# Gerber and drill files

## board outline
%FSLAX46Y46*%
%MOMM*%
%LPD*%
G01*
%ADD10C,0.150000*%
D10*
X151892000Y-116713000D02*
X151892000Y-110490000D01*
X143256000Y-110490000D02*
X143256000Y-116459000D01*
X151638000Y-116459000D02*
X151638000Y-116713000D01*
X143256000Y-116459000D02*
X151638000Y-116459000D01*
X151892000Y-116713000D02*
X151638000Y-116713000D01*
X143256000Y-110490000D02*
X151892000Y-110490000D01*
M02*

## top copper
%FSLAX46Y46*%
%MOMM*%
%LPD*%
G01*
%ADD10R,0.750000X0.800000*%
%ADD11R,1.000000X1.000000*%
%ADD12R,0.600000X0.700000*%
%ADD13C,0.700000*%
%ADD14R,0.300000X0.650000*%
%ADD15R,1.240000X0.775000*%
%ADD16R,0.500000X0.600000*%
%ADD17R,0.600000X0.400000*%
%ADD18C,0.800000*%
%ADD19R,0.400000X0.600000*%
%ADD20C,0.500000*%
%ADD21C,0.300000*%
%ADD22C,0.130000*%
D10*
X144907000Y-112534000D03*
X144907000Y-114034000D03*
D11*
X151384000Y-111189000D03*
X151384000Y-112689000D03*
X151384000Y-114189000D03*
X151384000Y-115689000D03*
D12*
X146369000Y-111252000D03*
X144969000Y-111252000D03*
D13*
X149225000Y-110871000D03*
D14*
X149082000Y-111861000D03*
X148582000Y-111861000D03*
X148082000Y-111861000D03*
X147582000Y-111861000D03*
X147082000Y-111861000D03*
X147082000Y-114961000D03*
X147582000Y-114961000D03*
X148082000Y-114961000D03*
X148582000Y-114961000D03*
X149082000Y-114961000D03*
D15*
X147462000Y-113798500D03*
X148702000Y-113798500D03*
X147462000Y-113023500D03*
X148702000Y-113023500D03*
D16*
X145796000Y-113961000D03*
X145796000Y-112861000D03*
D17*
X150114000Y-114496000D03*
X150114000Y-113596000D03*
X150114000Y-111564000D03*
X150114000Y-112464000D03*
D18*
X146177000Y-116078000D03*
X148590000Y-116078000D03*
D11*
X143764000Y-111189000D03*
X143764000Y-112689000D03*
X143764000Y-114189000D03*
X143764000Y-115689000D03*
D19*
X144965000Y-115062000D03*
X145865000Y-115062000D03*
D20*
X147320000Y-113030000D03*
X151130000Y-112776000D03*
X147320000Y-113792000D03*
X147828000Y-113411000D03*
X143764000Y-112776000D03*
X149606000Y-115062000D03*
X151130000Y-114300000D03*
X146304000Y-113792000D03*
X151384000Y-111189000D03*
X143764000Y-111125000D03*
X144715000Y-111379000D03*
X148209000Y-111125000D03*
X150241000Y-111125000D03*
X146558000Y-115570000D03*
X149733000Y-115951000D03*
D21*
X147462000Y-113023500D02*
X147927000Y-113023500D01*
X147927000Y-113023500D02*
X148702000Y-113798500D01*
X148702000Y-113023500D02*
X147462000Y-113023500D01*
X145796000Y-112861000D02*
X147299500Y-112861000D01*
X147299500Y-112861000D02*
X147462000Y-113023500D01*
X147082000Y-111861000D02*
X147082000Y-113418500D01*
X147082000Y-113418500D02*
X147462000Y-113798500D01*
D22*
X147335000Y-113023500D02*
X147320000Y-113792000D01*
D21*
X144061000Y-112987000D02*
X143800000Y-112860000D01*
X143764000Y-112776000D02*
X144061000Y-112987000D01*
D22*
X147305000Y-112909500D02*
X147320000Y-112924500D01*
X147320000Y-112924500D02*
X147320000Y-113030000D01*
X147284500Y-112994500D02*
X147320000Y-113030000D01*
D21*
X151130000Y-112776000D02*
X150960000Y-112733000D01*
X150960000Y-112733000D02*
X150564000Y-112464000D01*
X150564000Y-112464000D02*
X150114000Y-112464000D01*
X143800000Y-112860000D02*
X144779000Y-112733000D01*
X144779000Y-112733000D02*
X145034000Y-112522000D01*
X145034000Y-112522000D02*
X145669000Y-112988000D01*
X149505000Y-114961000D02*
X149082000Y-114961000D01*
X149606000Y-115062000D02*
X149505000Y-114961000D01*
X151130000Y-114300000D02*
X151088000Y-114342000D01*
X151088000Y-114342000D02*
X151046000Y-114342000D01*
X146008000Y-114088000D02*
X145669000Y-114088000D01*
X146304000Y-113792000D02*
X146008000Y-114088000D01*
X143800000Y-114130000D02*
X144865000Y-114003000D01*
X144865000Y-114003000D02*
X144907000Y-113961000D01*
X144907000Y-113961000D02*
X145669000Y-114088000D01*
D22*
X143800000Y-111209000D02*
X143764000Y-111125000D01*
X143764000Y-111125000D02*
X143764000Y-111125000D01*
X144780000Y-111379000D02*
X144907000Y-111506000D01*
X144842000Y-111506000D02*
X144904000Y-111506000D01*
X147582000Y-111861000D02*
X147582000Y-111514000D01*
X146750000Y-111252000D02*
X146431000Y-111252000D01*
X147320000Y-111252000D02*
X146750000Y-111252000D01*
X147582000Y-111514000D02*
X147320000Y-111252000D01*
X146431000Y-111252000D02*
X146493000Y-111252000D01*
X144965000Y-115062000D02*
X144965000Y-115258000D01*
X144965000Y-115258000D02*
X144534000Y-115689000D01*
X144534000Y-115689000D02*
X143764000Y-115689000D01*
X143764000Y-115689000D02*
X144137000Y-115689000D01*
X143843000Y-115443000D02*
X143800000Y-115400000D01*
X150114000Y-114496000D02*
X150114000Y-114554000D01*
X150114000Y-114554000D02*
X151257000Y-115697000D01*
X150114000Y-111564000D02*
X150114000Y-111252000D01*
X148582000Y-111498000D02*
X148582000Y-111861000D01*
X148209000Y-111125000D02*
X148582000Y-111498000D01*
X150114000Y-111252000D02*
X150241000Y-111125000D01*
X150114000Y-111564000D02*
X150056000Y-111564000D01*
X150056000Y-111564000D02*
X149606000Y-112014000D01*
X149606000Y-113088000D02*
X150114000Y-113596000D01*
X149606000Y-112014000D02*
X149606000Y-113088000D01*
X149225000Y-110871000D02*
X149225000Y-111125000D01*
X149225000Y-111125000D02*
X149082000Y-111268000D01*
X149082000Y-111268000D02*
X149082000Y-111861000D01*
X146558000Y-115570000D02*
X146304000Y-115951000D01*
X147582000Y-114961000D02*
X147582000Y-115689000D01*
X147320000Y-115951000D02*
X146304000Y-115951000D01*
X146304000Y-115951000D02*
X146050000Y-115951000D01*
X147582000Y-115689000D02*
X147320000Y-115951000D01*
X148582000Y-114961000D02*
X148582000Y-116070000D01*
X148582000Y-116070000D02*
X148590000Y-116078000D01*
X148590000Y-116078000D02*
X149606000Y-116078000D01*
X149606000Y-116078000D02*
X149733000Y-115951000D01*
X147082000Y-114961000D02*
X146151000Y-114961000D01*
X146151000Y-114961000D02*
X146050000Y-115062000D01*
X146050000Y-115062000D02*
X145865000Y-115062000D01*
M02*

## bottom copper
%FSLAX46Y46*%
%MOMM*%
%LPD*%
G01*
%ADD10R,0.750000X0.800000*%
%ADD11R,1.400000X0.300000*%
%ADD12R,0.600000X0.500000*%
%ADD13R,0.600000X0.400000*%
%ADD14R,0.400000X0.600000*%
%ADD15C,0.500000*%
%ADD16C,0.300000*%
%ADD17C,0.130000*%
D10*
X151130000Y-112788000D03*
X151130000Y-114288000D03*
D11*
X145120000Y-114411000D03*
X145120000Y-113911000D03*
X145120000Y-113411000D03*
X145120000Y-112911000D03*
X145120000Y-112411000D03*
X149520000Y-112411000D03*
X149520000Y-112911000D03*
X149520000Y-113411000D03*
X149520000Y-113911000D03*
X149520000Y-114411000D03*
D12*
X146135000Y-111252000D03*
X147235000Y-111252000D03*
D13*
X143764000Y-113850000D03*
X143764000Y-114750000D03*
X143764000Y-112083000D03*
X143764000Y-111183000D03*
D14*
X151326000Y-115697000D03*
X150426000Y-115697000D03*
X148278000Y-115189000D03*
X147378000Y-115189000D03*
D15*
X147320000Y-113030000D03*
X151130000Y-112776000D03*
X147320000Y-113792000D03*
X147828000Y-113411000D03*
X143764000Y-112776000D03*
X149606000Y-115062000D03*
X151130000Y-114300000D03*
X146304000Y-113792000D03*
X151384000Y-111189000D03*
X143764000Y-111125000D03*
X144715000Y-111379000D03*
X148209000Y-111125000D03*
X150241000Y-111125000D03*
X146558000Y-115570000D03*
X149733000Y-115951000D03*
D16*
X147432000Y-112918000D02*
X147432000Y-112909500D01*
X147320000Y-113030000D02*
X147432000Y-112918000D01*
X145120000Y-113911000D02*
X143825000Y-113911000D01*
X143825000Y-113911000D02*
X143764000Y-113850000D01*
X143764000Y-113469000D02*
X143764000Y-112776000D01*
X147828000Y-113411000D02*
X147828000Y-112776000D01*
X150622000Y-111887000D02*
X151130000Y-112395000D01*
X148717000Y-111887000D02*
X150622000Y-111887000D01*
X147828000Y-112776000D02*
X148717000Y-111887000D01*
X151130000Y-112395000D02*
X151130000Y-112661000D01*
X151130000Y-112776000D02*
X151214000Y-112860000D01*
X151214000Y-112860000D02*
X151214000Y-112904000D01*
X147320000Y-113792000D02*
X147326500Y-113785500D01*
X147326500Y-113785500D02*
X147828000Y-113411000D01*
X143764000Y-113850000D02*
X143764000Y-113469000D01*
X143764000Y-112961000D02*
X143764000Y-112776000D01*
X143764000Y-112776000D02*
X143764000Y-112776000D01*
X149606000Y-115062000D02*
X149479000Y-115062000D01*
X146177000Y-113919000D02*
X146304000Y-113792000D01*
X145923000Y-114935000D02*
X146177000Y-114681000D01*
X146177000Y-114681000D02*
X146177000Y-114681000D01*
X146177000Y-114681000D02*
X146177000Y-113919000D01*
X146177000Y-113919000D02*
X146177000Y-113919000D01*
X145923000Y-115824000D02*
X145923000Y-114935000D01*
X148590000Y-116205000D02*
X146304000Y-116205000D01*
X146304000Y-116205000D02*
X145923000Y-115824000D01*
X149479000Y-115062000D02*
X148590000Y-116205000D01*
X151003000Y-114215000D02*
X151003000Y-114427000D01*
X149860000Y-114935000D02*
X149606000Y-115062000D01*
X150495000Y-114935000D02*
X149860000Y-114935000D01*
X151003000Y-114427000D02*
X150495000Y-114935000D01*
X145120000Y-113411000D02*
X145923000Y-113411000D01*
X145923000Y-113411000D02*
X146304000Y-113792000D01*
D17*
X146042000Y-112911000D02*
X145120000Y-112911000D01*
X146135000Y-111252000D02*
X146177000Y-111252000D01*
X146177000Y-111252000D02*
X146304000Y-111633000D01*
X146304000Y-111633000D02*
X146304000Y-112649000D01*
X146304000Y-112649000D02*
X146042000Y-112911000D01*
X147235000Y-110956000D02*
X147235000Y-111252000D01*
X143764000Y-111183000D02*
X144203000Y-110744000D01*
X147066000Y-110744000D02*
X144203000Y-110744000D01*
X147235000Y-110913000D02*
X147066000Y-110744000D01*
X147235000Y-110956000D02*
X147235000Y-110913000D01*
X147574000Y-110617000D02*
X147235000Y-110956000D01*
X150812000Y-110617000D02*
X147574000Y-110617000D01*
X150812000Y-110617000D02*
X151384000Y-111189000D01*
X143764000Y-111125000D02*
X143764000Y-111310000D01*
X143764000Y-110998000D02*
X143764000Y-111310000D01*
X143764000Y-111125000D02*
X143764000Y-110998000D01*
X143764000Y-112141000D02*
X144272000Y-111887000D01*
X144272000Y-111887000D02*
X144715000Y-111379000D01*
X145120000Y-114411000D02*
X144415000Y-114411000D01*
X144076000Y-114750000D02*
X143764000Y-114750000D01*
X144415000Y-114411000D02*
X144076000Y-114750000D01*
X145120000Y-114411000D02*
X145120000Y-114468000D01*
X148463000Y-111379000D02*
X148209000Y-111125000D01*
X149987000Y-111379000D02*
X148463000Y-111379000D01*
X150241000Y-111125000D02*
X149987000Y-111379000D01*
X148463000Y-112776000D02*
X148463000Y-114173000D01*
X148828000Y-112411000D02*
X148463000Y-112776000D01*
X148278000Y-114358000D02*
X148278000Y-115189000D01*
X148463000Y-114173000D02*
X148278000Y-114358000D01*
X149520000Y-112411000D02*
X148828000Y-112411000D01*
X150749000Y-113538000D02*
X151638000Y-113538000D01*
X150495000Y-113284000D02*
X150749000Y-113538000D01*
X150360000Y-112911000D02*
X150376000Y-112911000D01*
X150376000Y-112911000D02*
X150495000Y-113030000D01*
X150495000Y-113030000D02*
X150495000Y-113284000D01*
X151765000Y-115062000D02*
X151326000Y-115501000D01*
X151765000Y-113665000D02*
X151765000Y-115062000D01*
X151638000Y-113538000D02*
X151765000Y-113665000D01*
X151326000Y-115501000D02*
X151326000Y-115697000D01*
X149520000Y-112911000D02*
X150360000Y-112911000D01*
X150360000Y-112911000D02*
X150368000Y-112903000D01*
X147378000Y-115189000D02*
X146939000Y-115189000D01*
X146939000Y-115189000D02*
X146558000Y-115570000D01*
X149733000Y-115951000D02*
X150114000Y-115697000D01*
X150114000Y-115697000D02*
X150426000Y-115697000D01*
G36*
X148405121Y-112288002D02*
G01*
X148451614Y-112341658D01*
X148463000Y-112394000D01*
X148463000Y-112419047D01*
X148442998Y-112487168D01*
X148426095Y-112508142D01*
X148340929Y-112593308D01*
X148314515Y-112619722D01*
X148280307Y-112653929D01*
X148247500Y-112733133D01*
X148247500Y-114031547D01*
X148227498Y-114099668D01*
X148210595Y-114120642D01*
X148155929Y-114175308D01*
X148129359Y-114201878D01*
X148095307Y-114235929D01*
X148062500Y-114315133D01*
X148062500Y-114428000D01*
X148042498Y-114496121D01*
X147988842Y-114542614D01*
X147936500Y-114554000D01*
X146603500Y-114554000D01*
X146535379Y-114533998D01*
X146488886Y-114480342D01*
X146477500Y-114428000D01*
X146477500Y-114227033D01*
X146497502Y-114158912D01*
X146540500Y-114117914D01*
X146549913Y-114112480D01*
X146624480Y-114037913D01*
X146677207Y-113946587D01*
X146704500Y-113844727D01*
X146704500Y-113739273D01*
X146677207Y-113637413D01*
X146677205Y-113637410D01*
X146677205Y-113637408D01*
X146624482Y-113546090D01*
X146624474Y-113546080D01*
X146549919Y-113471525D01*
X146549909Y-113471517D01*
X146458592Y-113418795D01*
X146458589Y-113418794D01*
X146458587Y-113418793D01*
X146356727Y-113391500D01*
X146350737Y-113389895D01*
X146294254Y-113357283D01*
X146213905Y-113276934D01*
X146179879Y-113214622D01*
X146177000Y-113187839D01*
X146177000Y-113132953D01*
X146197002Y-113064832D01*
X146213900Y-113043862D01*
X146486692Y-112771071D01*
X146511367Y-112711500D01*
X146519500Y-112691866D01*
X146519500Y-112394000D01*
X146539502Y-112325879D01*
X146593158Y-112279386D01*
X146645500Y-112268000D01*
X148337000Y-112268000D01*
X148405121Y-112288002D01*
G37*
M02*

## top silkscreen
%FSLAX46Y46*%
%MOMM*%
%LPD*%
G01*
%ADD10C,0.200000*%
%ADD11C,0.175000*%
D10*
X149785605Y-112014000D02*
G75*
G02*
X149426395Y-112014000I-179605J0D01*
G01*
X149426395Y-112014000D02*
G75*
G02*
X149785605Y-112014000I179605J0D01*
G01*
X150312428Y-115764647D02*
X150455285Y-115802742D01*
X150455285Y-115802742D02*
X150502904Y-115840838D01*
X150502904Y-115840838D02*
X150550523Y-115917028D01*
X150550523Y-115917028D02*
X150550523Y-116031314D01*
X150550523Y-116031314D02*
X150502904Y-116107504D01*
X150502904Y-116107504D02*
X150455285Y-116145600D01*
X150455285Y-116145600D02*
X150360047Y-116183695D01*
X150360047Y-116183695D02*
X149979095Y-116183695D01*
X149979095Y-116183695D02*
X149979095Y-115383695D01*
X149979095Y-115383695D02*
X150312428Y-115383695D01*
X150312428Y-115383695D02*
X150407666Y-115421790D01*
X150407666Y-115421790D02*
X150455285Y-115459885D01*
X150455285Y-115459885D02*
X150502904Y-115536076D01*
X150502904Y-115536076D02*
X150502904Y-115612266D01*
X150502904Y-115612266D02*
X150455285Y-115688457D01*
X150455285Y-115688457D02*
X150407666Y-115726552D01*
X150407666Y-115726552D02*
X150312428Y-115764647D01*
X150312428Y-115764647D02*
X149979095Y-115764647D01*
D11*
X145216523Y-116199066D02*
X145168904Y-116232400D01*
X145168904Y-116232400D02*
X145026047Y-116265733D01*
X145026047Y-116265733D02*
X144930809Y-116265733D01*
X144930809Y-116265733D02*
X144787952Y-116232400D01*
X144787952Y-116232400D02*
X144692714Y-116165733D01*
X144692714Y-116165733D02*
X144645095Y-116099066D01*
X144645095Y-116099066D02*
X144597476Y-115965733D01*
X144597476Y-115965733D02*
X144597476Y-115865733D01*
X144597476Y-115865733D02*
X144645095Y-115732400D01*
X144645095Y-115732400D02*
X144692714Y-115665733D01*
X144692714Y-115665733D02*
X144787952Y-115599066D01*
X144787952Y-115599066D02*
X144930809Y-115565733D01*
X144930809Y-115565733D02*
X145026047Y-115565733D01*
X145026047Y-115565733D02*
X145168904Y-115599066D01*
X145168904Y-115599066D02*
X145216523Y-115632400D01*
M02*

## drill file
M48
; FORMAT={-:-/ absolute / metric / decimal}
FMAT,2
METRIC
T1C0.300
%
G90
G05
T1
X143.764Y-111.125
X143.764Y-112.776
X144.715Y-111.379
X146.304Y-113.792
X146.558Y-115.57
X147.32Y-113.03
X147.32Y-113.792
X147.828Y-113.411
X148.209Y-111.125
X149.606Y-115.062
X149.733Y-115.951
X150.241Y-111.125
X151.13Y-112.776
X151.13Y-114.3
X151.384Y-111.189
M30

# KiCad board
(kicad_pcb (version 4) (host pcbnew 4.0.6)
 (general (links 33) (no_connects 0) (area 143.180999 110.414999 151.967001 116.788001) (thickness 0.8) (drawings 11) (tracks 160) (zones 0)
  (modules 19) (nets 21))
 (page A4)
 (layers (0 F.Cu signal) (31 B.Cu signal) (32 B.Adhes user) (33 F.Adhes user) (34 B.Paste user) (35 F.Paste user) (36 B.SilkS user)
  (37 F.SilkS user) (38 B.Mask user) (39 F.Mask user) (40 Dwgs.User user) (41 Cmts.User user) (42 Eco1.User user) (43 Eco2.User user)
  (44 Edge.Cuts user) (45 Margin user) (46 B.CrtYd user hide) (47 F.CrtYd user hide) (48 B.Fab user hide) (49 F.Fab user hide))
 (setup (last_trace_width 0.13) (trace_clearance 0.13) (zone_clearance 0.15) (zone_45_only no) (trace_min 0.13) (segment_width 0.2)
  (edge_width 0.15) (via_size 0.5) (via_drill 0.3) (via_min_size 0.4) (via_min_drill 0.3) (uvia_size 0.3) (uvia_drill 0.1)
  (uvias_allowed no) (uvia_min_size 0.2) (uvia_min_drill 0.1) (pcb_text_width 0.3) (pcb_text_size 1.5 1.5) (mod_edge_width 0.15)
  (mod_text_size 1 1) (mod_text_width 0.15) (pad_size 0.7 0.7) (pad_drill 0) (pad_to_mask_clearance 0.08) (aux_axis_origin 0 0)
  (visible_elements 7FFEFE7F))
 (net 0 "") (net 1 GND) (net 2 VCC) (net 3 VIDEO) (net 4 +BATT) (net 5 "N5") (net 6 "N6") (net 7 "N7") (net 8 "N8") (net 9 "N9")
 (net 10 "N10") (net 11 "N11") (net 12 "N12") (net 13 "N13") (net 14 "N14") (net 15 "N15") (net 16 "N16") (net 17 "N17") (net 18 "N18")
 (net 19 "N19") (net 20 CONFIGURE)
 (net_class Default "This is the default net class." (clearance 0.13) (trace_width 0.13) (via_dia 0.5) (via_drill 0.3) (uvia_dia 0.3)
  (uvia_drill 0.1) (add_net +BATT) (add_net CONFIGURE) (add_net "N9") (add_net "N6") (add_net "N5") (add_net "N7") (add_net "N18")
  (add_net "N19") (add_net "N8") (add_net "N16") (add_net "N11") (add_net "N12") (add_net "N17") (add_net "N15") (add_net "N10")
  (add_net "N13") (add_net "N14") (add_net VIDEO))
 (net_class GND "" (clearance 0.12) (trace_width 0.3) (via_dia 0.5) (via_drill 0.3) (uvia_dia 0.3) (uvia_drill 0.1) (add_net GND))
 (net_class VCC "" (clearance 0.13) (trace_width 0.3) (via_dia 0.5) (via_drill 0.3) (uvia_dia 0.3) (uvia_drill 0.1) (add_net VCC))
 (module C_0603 (layer B.Cu) (at 151.13 113.538 270)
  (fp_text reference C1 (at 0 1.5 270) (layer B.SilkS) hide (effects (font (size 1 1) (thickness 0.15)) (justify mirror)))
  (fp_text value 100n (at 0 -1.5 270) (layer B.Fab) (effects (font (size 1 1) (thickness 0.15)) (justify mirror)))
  (pad 1 smd rect (at -0.75 0 270) (size 0.8 0.75) (layers B.Cu B.Paste B.Mask) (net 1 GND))
  (pad 2 smd rect (at 0.75 0 270) (size 0.8 0.75) (layers B.Cu B.Paste B.Mask) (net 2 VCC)))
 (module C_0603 (layer F.Cu) (at 144.907 113.284 270)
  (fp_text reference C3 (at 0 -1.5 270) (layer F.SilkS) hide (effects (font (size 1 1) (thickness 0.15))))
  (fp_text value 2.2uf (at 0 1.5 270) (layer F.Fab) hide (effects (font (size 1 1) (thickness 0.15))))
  (pad 1 smd rect (at -0.75 0 270) (size 0.8 0.75) (layers F.Cu F.Paste F.Mask) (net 1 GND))
  (pad 2 smd rect (at 0.75 0 270) (size 0.8 0.75) (layers F.Cu F.Paste F.Mask) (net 2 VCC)))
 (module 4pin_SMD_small (layer F.Cu) (at 151.384 115.189 90)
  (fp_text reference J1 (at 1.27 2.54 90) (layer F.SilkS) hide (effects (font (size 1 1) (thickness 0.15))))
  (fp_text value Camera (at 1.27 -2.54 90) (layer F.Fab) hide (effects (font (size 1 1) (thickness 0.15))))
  (pad 4 smd rect (at 4 0 90) (size 1 1) (layers F.Cu F.Paste F.Mask) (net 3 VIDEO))
  (pad 3 smd rect (at 2.5 0 90) (size 1 1) (layers F.Cu F.Paste F.Mask) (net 1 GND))
  (pad 2 smd rect (at 1 0 90) (size 1 1) (layers F.Cu F.Paste F.Mask) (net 2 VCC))
  (pad 1 smd rect (at -0.5 0 90) (size 1 1) (layers F.Cu F.Paste F.Mask) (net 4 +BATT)))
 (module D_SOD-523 (layer F.Cu) (at 145.669 111.252)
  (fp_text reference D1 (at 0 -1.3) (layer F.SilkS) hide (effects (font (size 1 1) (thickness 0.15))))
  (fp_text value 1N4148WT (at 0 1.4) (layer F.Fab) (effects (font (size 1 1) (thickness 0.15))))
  (pad 2 smd rect (at 0.7 0 180) (size 0.6 0.7) (layers F.Cu F.Paste F.Mask) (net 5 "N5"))
  (pad 1 smd rect (at -0.7 0 180) (size 0.6 0.7) (layers F.Cu F.Paste F.Mask) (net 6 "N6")))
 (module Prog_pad (layer F.Cu) (at 149.225 110.871)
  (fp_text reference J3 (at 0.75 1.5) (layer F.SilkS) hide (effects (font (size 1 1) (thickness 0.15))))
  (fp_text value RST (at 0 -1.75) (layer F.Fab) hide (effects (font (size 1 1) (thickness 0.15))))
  (pad 1 smd circle (at 0 0) (size 0.7 0.7) (layers F.Cu F.Paste F.Mask) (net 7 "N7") (solder_mask_margin 0.02)))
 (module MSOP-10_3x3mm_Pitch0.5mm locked (layer B.Cu) (at 147.32 113.411)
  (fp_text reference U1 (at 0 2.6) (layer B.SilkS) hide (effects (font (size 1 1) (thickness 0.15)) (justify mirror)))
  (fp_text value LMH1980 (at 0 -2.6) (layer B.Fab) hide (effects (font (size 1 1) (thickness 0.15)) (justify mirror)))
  (pad 1 smd rect (at -2.2 1) (size 1.4 0.3) (layers B.Cu B.Paste B.Mask) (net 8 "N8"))
  (pad 2 smd rect (at -2.2 0.5) (size 1.4 0.3) (layers B.Cu B.Paste B.Mask) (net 1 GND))
  (pad 3 smd rect (at -2.2 0) (size 1.4 0.3) (layers B.Cu B.Paste B.Mask) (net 2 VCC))
  (pad 4 smd rect (at -2.2 -0.5) (size 1.4 0.3) (layers B.Cu B.Paste B.Mask) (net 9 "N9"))
  (pad 5 smd rect (at -2.2 -1) (size 1.4 0.3) (layers B.Cu B.Paste B.Mask) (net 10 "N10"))
  (pad 6 smd rect (at 2.2 -1) (size 1.4 0.3) (layers B.Cu B.Paste B.Mask) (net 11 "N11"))
  (pad 7 smd rect (at 2.2 -0.5) (size 1.4 0.3) (layers B.Cu B.Paste B.Mask) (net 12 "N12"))
  (pad 8 smd rect (at 2.2 0) (size 1.4 0.3) (layers B.Cu B.Paste B.Mask) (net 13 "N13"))
  (pad 9 smd rect (at 2.2 0.5) (size 1.4 0.3) (layers B.Cu B.Paste B.Mask) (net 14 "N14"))
  (pad 10 smd rect (at 2.2 1) (size 1.4 0.3) (layers B.Cu B.Paste B.Mask) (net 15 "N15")))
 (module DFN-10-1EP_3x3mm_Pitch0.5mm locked (layer F.Cu) (at 148.082 113.411 270)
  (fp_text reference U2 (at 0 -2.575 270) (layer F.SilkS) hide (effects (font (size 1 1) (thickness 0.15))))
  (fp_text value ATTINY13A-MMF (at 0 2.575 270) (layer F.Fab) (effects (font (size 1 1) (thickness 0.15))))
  (pad 1 smd rect (at -1.55 -1 270) (size 0.65 0.3) (layers F.Cu F.Paste F.Mask) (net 7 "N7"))
  (pad 2 smd rect (at -1.55 -0.5 270) (size 0.65 0.3) (layers F.Cu F.Paste F.Mask) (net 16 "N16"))
  (pad 3 smd rect (at -1.55 0 270) (size 0.65 0.3) (layers F.Cu F.Paste F.Mask))
  (pad 4 smd rect (at -1.55 0.5 270) (size 0.65 0.3) (layers F.Cu F.Paste F.Mask) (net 5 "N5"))
  (pad 5 smd rect (at -1.55 1 270) (size 0.65 0.3) (layers F.Cu F.Paste F.Mask) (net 1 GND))
  (pad 6 smd rect (at 1.55 1 270) (size 0.65 0.3) (layers F.Cu F.Paste F.Mask) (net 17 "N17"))
  (pad 7 smd rect (at 1.55 0.5 270) (size 0.65 0.3) (layers F.Cu F.Paste F.Mask) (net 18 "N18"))
  (pad 8 smd rect (at 1.55 0 270) (size 0.65 0.3) (layers F.Cu F.Paste F.Mask))
  (pad 9 smd rect (at 1.55 -0.5 270) (size 0.65 0.3) (layers F.Cu F.Paste F.Mask) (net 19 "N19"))
  (pad 10 smd rect (at 1.55 -1 270) (size 0.65 0.3) (layers F.Cu F.Paste F.Mask) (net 2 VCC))
  (pad 11 smd rect (at 0.3875 0.62 270) (size 0.775 1.24) (layers F.Cu F.Paste F.Mask) (solder_paste_margin_ratio -0.2))
  (pad 11 smd rect (at 0.3875 -0.62 270) (size 0.775 1.24) (layers F.Cu F.Paste F.Mask) (solder_paste_margin_ratio -0.2))
  (pad 11 smd rect (at -0.3875 0.62 270) (size 0.775 1.24) (layers F.Cu F.Paste F.Mask) (solder_paste_margin_ratio -0.2))
  (pad 11 smd rect (at -0.3875 -0.62 270) (size 0.775 1.24) (layers F.Cu F.Paste F.Mask) (solder_paste_margin_ratio -0.2)))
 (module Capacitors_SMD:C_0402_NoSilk (layer B.Cu) (at 146.685 111.252)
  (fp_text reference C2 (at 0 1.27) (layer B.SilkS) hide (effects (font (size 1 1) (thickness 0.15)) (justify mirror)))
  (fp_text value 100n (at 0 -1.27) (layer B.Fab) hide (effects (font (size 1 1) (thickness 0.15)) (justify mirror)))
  (pad 1 smd rect (at -0.55 0) (size 0.6 0.5) (layers B.Cu B.Paste B.Mask) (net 9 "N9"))
  (pad 2 smd rect (at 0.55 0) (size 0.6 0.5) (layers B.Cu B.Paste B.Mask) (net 3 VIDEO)))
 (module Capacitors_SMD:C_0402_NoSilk (layer F.Cu) (at 145.796 113.411 90)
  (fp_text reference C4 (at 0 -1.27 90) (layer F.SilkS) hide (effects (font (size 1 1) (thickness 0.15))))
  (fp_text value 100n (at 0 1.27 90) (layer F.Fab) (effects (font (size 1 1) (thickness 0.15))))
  (pad 1 smd rect (at -0.55 0 90) (size 0.6 0.5) (layers F.Cu F.Paste F.Mask) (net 2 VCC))
  (pad 2 smd rect (at 0.55 0 90) (size 0.6 0.5) (layers F.Cu F.Paste F.Mask) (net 1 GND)))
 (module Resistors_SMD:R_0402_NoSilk (layer B.Cu) (at 143.764 114.3 270)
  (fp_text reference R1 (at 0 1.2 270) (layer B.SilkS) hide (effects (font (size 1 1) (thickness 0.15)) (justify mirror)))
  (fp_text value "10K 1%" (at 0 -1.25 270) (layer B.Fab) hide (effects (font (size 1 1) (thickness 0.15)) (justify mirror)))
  (pad 1 smd rect (at -0.45 0 270) (size 0.4 0.6) (layers B.Cu B.Paste B.Mask) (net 1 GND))
  (pad 2 smd rect (at 0.45 0 270) (size 0.4 0.6) (layers B.Cu B.Paste B.Mask) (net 8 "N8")))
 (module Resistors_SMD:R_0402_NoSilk (layer B.Cu) (at 143.764 111.633 90)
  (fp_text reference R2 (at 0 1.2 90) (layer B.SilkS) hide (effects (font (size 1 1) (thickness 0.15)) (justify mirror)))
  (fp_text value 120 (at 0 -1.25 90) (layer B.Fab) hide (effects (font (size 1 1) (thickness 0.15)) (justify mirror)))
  (pad 1 smd rect (at -0.45 0 90) (size 0.4 0.6) (layers B.Cu B.Paste B.Mask) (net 6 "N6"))
  (pad 2 smd rect (at 0.45 0 90) (size 0.4 0.6) (layers B.Cu B.Paste B.Mask) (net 3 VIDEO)))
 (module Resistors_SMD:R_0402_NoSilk (layer F.Cu) (at 150.114 114.046 90)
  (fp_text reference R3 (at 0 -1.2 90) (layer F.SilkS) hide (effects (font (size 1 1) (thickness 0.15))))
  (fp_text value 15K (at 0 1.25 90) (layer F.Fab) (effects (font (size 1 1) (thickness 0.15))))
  (pad 1 smd rect (at -0.45 0 90) (size 0.4 0.6) (layers F.Cu F.Paste F.Mask) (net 4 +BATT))
  (pad 2 smd rect (at 0.45 0 90) (size 0.4 0.6) (layers F.Cu F.Paste F.Mask) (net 16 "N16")))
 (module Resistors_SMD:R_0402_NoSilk (layer F.Cu) (at 150.114 112.014 270)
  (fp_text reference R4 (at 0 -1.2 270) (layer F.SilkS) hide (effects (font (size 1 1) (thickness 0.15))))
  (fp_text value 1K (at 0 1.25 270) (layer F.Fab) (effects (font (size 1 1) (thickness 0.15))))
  (pad 1 smd rect (at -0.45 0 270) (size 0.4 0.6) (layers F.Cu F.Paste F.Mask) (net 16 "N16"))
  (pad 2 smd rect (at 0.45 0 270) (size 0.4 0.6) (layers F.Cu F.Paste F.Mask) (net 1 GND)))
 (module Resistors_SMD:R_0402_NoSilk (layer B.Cu) (at 150.876 115.697 180)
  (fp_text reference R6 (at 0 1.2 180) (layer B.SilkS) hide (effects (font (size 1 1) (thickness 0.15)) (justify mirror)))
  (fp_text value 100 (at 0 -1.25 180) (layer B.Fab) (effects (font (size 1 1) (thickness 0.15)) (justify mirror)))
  (pad 1 smd rect (at -0.45 0 180) (size 0.4 0.6) (layers B.Cu B.Paste B.Mask) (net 12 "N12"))
  (pad 2 smd rect (at 0.45 0 180) (size 0.4 0.6) (layers B.Cu B.Paste B.Mask) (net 19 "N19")))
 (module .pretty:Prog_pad (layer F.Cu) (at 146.177 116.078)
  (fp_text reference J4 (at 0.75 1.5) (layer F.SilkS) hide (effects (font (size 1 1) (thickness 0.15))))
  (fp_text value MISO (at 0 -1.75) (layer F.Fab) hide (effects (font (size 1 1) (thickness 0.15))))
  (pad 1 smd circle (at 0 0) (size 0.8 0.8) (layers F.Cu F.Paste F.Mask) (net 18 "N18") (solder_mask_margin 0.02)))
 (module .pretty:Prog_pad (layer F.Cu) (at 148.59 116.078)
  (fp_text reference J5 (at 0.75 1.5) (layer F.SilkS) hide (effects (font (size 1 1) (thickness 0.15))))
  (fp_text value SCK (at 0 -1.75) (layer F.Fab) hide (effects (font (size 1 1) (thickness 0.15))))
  (pad 1 smd circle (at 0 0) (size 0.8 0.8) (layers F.Cu F.Paste F.Mask) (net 19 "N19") (solder_mask_margin 0.02)))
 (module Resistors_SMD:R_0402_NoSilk (layer B.Cu) (at 147.828 115.189 180)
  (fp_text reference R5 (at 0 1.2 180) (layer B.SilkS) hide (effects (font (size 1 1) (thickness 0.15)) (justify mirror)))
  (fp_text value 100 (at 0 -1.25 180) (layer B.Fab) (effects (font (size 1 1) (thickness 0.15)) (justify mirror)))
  (pad 1 smd rect (at -0.45 0 180) (size 0.4 0.6) (layers B.Cu B.Paste B.Mask) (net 11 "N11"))
  (pad 2 smd rect (at 0.45 0 180) (size 0.4 0.6) (layers B.Cu B.Paste B.Mask) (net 18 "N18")))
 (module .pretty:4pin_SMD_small (layer F.Cu) (at 143.764 115.189 90)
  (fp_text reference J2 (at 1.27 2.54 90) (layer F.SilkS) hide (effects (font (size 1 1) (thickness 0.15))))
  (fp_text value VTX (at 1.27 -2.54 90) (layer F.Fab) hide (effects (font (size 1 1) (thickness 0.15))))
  (pad 4 smd rect (at 4 0 90) (size 1 1) (layers F.Cu F.Paste F.Mask) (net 3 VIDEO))
  (pad 3 smd rect (at 2.5 0 90) (size 1 1) (layers F.Cu F.Paste F.Mask) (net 1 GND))
  (pad 2 smd rect (at 1 0 90) (size 1 1) (layers F.Cu F.Paste F.Mask) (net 2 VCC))
  (pad 1 smd rect (at -0.5 0 90) (size 1 1) (layers F.Cu F.Paste F.Mask) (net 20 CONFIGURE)))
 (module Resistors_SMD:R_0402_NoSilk (layer F.Cu) (at 145.415 115.062)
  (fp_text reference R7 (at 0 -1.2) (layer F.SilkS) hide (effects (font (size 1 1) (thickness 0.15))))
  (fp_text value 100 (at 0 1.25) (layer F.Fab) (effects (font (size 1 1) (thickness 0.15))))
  (pad 1 smd rect (at -0.45 0) (size 0.4 0.6) (layers F.Cu F.Paste F.Mask) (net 20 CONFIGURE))
  (pad 2 smd rect (at 0.45 0) (size 0.4 0.6) (layers F.Cu F.Paste F.Mask) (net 17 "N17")))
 (gr_line (start 151.892 116.713) (end 151.892 110.49) (angle 90) (layer Edge.Cuts) (width 0.15))
 (gr_line (start 143.256 110.49) (end 143.256 116.459) (angle 90) (layer Edge.Cuts) (width 0.15))
 (gr_line (start 151.638 116.459) (end 151.638 116.713) (angle 90) (layer Edge.Cuts) (width 0.15))
 (gr_line (start 143.256 116.459) (end 151.638 116.459) (angle 90) (layer Edge.Cuts) (width 0.15))
 (gr_line (start 151.892 116.713) (end 151.638 116.713) (angle 90) (layer Edge.Cuts) (width 0.15))
 (gr_circle (center 149.606 112.014) (end 149.479 111.887) (layer F.SilkS) (width 0.2))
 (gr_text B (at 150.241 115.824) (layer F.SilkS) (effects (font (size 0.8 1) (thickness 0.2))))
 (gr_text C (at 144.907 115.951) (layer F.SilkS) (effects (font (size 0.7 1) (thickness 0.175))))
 (gr_line (start 143.256 110.49) (end 151.892 110.49) (angle 90) (layer Edge.Cuts) (width 0.15))
 (segment (start 147.462 113.0235) (end 147.927 113.0235) (width 0.3) (layer F.Cu) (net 1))
 (segment (start 147.927 113.0235) (end 148.702 113.7985) (width 0.3) (layer F.Cu) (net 1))
 (segment (start 148.702 113.0235) (end 147.462 113.0235) (width 0.3) (layer F.Cu) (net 1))
 (segment (start 145.796 112.861) (end 147.2995 112.861) (width 0.3) (layer F.Cu) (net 1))
 (segment (start 147.2995 112.861) (end 147.462 113.0235) (width 0.3) (layer F.Cu) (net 1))
 (segment (start 147.082 111.861) (end 147.082 113.4185) (width 0.3) (layer F.Cu) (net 1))
 (segment (start 147.082 113.4185) (end 147.462 113.7985) (width 0.3) (layer F.Cu) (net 1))
 (via (at 147.32 113.03) (size 0.5) (drill 0.3) (layers F.Cu B.Cu) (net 1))
 (segment (start 147.432 112.918) (end 147.432 112.9095) (width 0.3) (layer B.Cu) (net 1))
 (segment (start 147.32 113.03) (end 147.432 112.918) (width 0.3) (layer B.Cu) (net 1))
 (segment (start 145.12 113.911) (end 143.825 113.911) (width 0.3) (layer B.Cu) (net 1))
 (segment (start 143.825 113.911) (end 143.764 113.85) (width 0.3) (layer B.Cu) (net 1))
 (segment (start 143.764 113.469) (end 143.764 112.776) (width 0.3) (layer B.Cu) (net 1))
 (segment (start 147.828 113.411) (end 147.828 112.776) (width 0.3) (layer B.Cu) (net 1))
 (segment (start 150.622 111.887) (end 151.13 112.395) (width 0.3) (layer B.Cu) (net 1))
 (segment (start 148.717 111.887) (end 150.622 111.887) (width 0.3) (layer B.Cu) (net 1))
 (segment (start 147.828 112.776) (end 148.717 111.887) (width 0.3) (layer B.Cu) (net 1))
 (segment (start 151.13 112.395) (end 151.13 112.661) (width 0.3) (layer B.Cu) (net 1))
 (via (at 151.13 112.776) (size 0.5) (drill 0.3) (layers F.Cu B.Cu) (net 1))
 (segment (start 151.13 112.776) (end 151.214 112.86) (width 0.3) (layer B.Cu) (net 1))
 (segment (start 151.214 112.86) (end 151.214 112.904) (width 0.3) (layer B.Cu) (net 1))
 (segment (start 147.335 113.0235) (end 147.32 113.792) (width 0.13) (layer F.Cu) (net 1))
 (via (at 147.32 113.792) (size 0.5) (drill 0.3) (layers F.Cu B.Cu) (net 1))
 (segment (start 147.32 113.792) (end 147.3265 113.7855) (width 0.3) (layer B.Cu) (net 1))
 (segment (start 147.3265 113.7855) (end 147.828 113.411) (width 0.3) (layer B.Cu) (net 1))
 (via (at 147.828 113.411) (size 0.5) (drill 0.3) (layers F.Cu B.Cu) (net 1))
 (segment (start 143.764 113.85) (end 143.764 113.469) (width 0.3) (layer B.Cu) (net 1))
 (segment (start 143.764 112.961) (end 143.764 112.776) (width 0.3) (layer B.Cu) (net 1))
 (segment (start 144.061 112.987) (end 143.8 112.86) (width 0.3) (layer F.Cu) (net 1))
 (segment (start 143.764 112.776) (end 144.061 112.987) (width 0.3) (layer F.Cu) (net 1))
 (via (at 143.764 112.776) (size 0.5) (drill 0.3) (layers F.Cu B.Cu) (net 1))
 (segment (start 143.764 112.776) (end 143.764 112.776) (width 0.3) (layer B.Cu) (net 1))
 (segment (start 147.305 112.9095) (end 147.32 112.9245) (width 0.13) (layer F.Cu) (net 1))
 (segment (start 147.32 112.9245) (end 147.32 113.03) (width 0.13) (layer F.Cu) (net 1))
 (segment (start 147.2845 112.9945) (end 147.32 113.03) (width 0.13) (layer F.Cu) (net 1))
 (segment (start 151.13 112.776) (end 150.96 112.733) (width 0.3) (layer F.Cu) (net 1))
 (segment (start 150.96 112.733) (end 150.564 112.464) (width 0.3) (layer F.Cu) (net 1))
 (segment (start 150.564 112.464) (end 150.114 112.464) (width 0.3) (layer F.Cu) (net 1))
 (segment (start 143.8 112.86) (end 144.779 112.733) (width 0.3) (layer F.Cu) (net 1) (status 20))
 (segment (start 144.779 112.733) (end 145.034 112.522) (width 0.3) (layer F.Cu) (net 1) (status 30))
 (segment (start 145.034 112.522) (end 145.669 112.988) (width 0.3) (layer F.Cu) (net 1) (status 10))
 (segment (start 149.606 115.062) (end 149.479 115.062) (width 0.3) (layer B.Cu) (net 2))
 (segment (start 146.177 113.919) (end 146.304 113.792) (width 0.3) (layer B.Cu) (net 2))
 (segment (start 145.923 114.935) (end 146.177 114.681) (width 0.3) (layer B.Cu) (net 2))
 (segment (start 146.177 114.681) (end 146.177 114.681) (width 0.3) (layer B.Cu) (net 2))
 (segment (start 146.177 114.681) (end 146.177 113.919) (width 0.3) (layer B.Cu) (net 2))
 (segment (start 146.177 113.919) (end 146.177 113.919) (width 0.3) (layer B.Cu) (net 2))
 (segment (start 145.923 115.824) (end 145.923 114.935) (width 0.3) (layer B.Cu) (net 2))
 (segment (start 148.59 116.205) (end 146.304 116.205) (width 0.3) (layer B.Cu) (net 2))
 (segment (start 146.304 116.205) (end 145.923 115.824) (width 0.3) (layer B.Cu) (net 2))
 (segment (start 149.479 115.062) (end 148.59 116.205) (width 0.3) (layer B.Cu) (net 2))
 (segment (start 151.003 114.215) (end 151.003 114.427) (width 0.3) (layer B.Cu) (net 2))
 (segment (start 149.505 114.961) (end 149.082 114.961) (width 0.3) (layer F.Cu) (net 2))
 (segment (start 149.606 115.062) (end 149.505 114.961) (width 0.3) (layer F.Cu) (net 2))
 (via (at 149.606 115.062) (size 0.5) (drill 0.3) (layers F.Cu B.Cu) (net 2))
 (segment (start 149.86 114.935) (end 149.606 115.062) (width 0.3) (layer B.Cu) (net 2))
 (segment (start 150.495 114.935) (end 149.86 114.935) (width 0.3) (layer B.Cu) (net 2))
 (segment (start 151.003 114.427) (end 150.495 114.935) (width 0.3) (layer B.Cu) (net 2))
 (via (at 151.13 114.3) (size 0.5) (drill 0.3) (layers F.Cu B.Cu) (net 2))
 (segment (start 151.13 114.3) (end 151.088 114.342) (width 0.3) (layer F.Cu) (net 2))
 (segment (start 151.088 114.342) (end 151.046 114.342) (width 0.3) (layer F.Cu) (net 2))
 (segment (start 145.12 113.411) (end 145.923 113.411) (width 0.3) (layer B.Cu) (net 2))
 (segment (start 145.923 113.411) (end 146.304 113.792) (width 0.3) (layer B.Cu) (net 2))
 (segment (start 146.008 114.088) (end 145.669 114.088) (width 0.3) (layer F.Cu) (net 2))
 (segment (start 146.304 113.792) (end 146.008 114.088) (width 0.3) (layer F.Cu) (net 2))
 (via (at 146.304 113.792) (size 0.5) (drill 0.3) (layers F.Cu B.Cu) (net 2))
 (segment (start 143.8 114.13) (end 144.865 114.003) (width 0.3) (layer F.Cu) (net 2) (status 20))
 (segment (start 144.865 114.003) (end 144.907 113.961) (width 0.3) (layer F.Cu) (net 2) (status 30))
 (segment (start 144.907 113.961) (end 145.669 114.088) (width 0.3) (layer F.Cu) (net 2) (status 10))
 (segment (start 146.042 112.911) (end 145.12 112.911) (width 0.13) (layer B.Cu) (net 9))
 (segment (start 146.135 111.252) (end 146.177 111.252) (width 0.13) (layer B.Cu) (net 9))
 (segment (start 146.177 111.252) (end 146.304 111.633) (width 0.13) (layer B.Cu) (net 9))
 (segment (start 146.304 111.633) (end 146.304 112.649) (width 0.13) (layer B.Cu) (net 9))
 (segment (start 146.304 112.649) (end 146.042 112.911) (width 0.13) (layer B.Cu) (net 9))
 (segment (start 147.235 110.956) (end 147.235 111.252) (width 0.13) (layer B.Cu) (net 3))
 (via (at 151.384 111.189) (size 0.5) (drill 0.3) (layers F.Cu B.Cu) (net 3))
 (segment (start 143.764 111.183) (end 144.203 110.744) (width 0.13) (layer B.Cu) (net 3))
 (segment (start 147.066 110.744) (end 144.203 110.744) (width 0.13) (layer B.Cu) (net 3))
 (segment (start 147.235 110.913) (end 147.066 110.744) (width 0.13) (layer B.Cu) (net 3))
 (segment (start 147.235 110.956) (end 147.235 110.913) (width 0.13) (layer B.Cu) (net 3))
 (segment (start 147.574 110.617) (end 147.235 110.956) (width 0.13) (layer B.Cu) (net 3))
 (segment (start 150.812 110.617) (end 147.574 110.617) (width 0.13) (layer B.Cu) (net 3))
 (segment (start 150.812 110.617) (end 151.384 111.189) (width 0.13) (layer B.Cu) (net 3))
 (segment (start 143.764 111.125) (end 143.764 111.31) (width 0.13) (layer B.Cu) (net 3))
 (segment (start 143.8 111.209) (end 143.764 111.125) (width 0.13) (layer F.Cu) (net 3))
 (segment (start 143.764 110.998) (end 143.764 111.31) (width 0.13) (layer B.Cu) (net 3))
 (segment (start 143.764 111.125) (end 143.764 110.998) (width 0.13) (layer B.Cu) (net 3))
 (via (at 143.764 111.125) (size 0.5) (drill 0.3) (layers F.Cu B.Cu) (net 3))
 (segment (start 143.764 111.125) (end 143.764 111.125) (width 0.13) (layer F.Cu) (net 3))
 (via (at 144.715 111.379) (size 0.5) (drill 0.3) (layers F.Cu B.Cu) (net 6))
 (segment (start 144.78 111.379) (end 144.907 111.506) (width 0.13) (layer F.Cu) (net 6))
 (segment (start 144.842 111.506) (end 144.904 111.506) (width 0.13) (layer F.Cu) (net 6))
 (segment (start 143.764 112.141) (end 144.272 111.887) (width 0.13) (layer B.Cu) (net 6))
 (segment (start 144.272 111.887) (end 144.715 111.379) (width 0.13) (layer B.Cu) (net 6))
 (segment (start 147.582 111.861) (end 147.582 111.514) (width 0.13) (layer F.Cu) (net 5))
 (segment (start 146.75 111.252) (end 146.431 111.252) (width 0.13) (layer F.Cu) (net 5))
 (segment (start 147.32 111.252) (end 146.75 111.252) (width 0.13) (layer F.Cu) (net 5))
 (segment (start 147.582 111.514) (end 147.32 111.252) (width 0.13) (layer F.Cu) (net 5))
 (segment (start 146.431 111.252) (end 146.493 111.252) (width 0.13) (layer F.Cu) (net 5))
 (segment (start 144.965 115.062) (end 144.965 115.258) (width 0.13) (layer F.Cu) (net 20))
 (segment (start 144.965 115.258) (end 144.534 115.689) (width 0.13) (layer F.Cu) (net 20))
 (segment (start 144.534 115.689) (end 143.764 115.689) (width 0.13) (layer F.Cu) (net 20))
 (segment (start 143.764 115.689) (end 144.137 115.689) (width 0.13) (layer F.Cu) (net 20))
 (segment (start 143.843 115.443) (end 143.8 115.4) (width 0.13) (layer F.Cu) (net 20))
 (segment (start 150.114 114.496) (end 150.114 114.554) (width 0.13) (layer F.Cu) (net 4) (status 10))
 (segment (start 150.114 114.554) (end 151.257 115.697) (width 0.13) (layer F.Cu) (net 4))
 (segment (start 145.12 114.411) (end 144.415 114.411) (width 0.13) (layer B.Cu) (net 8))
 (segment (start 144.076 114.75) (end 143.764 114.75) (width 0.13) (layer B.Cu) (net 8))
 (segment (start 144.415 114.411) (end 144.076 114.75) (width 0.13) (layer B.Cu) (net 8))
 (segment (start 145.12 114.411) (end 145.12 114.468) (width 0.13) (layer B.Cu) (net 8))
 (segment (start 150.114 111.564) (end 150.114 111.252) (width 0.13) (layer F.Cu) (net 16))
 (segment (start 148.582 111.498) (end 148.582 111.861) (width 0.13) (layer F.Cu) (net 16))
 (segment (start 148.209 111.125) (end 148.582 111.498) (width 0.13) (layer F.Cu) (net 16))
 (via (at 148.209 111.125) (size 0.5) (drill 0.3) (layers F.Cu B.Cu) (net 16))
 (segment (start 148.463 111.379) (end 148.209 111.125) (width 0.13) (layer B.Cu) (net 16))
 (segment (start 149.987 111.379) (end 148.463 111.379) (width 0.13) (layer B.Cu) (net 16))
 (segment (start 150.241 111.125) (end 149.987 111.379) (width 0.13) (layer B.Cu) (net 16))
 (via (at 150.241 111.125) (size 0.5) (drill 0.3) (layers F.Cu B.Cu) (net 16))
 (segment (start 150.114 111.252) (end 150.241 111.125) (width 0.13) (layer F.Cu) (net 16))
 (segment (start 150.114 111.564) (end 150.056 111.564) (width 0.13) (layer F.Cu) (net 16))
 (segment (start 150.056 111.564) (end 149.606 112.014) (width 0.13) (layer F.Cu) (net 16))
 (segment (start 149.606 113.088) (end 150.114 113.596) (width 0.13) (layer F.Cu) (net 16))
 (segment (start 149.606 112.014) (end 149.606 113.088) (width 0.13) (layer F.Cu) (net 16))
 (segment (start 148.463 112.776) (end 148.463 114.173) (width 0.13) (layer B.Cu) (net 11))
 (segment (start 148.828 112.411) (end 148.463 112.776) (width 0.13) (layer B.Cu) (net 11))
 (segment (start 148.278 114.358) (end 148.278 115.189) (width 0.13) (layer B.Cu) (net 11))
 (segment (start 148.463 114.173) (end 148.278 114.358) (width 0.13) (layer B.Cu) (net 11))
 (segment (start 149.52 112.411) (end 148.828 112.411) (width 0.13) (layer B.Cu) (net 11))
 (segment (start 150.749 113.538) (end 151.638 113.538) (width 0.13) (layer B.Cu) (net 12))
 (segment (start 150.495 113.284) (end 150.749 113.538) (width 0.13) (layer B.Cu) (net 12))
 (segment (start 150.36 112.911) (end 150.376 112.911) (width 0.13) (layer B.Cu) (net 12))
 (segment (start 150.376 112.911) (end 150.495 113.03) (width 0.13) (layer B.Cu) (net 12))
 (segment (start 150.495 113.03) (end 150.495 113.284) (width 0.13) (layer B.Cu) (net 12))
 (segment (start 151.765 115.062) (end 151.326 115.501) (width 0.13) (layer B.Cu) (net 12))
 (segment (start 151.765 113.665) (end 151.765 115.062) (width 0.13) (layer B.Cu) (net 12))
 (segment (start 151.638 113.538) (end 151.765 113.665) (width 0.13) (layer B.Cu) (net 12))
 (segment (start 151.326 115.501) (end 151.326 115.697) (width 0.13) (layer B.Cu) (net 12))
 (segment (start 149.52 112.911) (end 150.36 112.911) (width 0.13) (layer B.Cu) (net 12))
 (segment (start 150.36 112.911) (end 150.368 112.903) (width 0.13) (layer B.Cu) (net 12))
 (segment (start 149.225 110.871) (end 149.225 111.125) (width 0.13) (layer F.Cu) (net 7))
 (segment (start 149.225 111.125) (end 149.082 111.268) (width 0.13) (layer F.Cu) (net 7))
 (segment (start 149.082 111.268) (end 149.082 111.861) (width 0.13) (layer F.Cu) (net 7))
 (segment (start 147.378 115.189) (end 146.939 115.189) (width 0.13) (layer B.Cu) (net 18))
 (segment (start 146.558 115.57) (end 146.304 115.951) (width 0.13) (layer F.Cu) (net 18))
 (via (at 146.558 115.57) (size 0.5) (drill 0.3) (layers F.Cu B.Cu) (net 18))
 (segment (start 146.939 115.189) (end 146.558 115.57) (width 0.13) (layer B.Cu) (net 18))
 (segment (start 147.582 114.961) (end 147.582 115.689) (width 0.13) (layer F.Cu) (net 18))
 (segment (start 147.32 115.951) (end 146.304 115.951) (width 0.13) (layer F.Cu) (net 18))
 (segment (start 146.304 115.951) (end 146.05 115.951) (width 0.13) (layer F.Cu) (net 18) (status 20))
 (segment (start 147.582 115.689) (end 147.32 115.951) (width 0.13) (layer F.Cu) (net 18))
 (segment (start 148.582 114.961) (end 148.582 116.07) (width 0.13) (layer F.Cu) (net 19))
 (segment (start 148.582 116.07) (end 148.59 116.078) (width 0.13) (layer F.Cu) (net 19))
 (segment (start 148.59 116.078) (end 149.606 116.078) (width 0.13) (layer F.Cu) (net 19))
 (segment (start 149.606 116.078) (end 149.733 115.951) (width 0.13) (layer F.Cu) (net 19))
 (via (at 149.733 115.951) (size 0.5) (drill 0.3) (layers F.Cu B.Cu) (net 19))
 (segment (start 149.733 115.951) (end 150.114 115.697) (width 0.13) (layer B.Cu) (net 19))
 (segment (start 150.114 115.697) (end 150.426 115.697) (width 0.13) (layer B.Cu) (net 19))
 (segment (start 147.082 114.961) (end 146.151 114.961) (width 0.13) (layer F.Cu) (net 17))
 (segment (start 146.151 114.961) (end 146.05 115.062) (width 0.13) (layer F.Cu) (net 17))
 (segment (start 146.05 115.062) (end 145.865 115.062) (width 0.13) (layer F.Cu) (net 17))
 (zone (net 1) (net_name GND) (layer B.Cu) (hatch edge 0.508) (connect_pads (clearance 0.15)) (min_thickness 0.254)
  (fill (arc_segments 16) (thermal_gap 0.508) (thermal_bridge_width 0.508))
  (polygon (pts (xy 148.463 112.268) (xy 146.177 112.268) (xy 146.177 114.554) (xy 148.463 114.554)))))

